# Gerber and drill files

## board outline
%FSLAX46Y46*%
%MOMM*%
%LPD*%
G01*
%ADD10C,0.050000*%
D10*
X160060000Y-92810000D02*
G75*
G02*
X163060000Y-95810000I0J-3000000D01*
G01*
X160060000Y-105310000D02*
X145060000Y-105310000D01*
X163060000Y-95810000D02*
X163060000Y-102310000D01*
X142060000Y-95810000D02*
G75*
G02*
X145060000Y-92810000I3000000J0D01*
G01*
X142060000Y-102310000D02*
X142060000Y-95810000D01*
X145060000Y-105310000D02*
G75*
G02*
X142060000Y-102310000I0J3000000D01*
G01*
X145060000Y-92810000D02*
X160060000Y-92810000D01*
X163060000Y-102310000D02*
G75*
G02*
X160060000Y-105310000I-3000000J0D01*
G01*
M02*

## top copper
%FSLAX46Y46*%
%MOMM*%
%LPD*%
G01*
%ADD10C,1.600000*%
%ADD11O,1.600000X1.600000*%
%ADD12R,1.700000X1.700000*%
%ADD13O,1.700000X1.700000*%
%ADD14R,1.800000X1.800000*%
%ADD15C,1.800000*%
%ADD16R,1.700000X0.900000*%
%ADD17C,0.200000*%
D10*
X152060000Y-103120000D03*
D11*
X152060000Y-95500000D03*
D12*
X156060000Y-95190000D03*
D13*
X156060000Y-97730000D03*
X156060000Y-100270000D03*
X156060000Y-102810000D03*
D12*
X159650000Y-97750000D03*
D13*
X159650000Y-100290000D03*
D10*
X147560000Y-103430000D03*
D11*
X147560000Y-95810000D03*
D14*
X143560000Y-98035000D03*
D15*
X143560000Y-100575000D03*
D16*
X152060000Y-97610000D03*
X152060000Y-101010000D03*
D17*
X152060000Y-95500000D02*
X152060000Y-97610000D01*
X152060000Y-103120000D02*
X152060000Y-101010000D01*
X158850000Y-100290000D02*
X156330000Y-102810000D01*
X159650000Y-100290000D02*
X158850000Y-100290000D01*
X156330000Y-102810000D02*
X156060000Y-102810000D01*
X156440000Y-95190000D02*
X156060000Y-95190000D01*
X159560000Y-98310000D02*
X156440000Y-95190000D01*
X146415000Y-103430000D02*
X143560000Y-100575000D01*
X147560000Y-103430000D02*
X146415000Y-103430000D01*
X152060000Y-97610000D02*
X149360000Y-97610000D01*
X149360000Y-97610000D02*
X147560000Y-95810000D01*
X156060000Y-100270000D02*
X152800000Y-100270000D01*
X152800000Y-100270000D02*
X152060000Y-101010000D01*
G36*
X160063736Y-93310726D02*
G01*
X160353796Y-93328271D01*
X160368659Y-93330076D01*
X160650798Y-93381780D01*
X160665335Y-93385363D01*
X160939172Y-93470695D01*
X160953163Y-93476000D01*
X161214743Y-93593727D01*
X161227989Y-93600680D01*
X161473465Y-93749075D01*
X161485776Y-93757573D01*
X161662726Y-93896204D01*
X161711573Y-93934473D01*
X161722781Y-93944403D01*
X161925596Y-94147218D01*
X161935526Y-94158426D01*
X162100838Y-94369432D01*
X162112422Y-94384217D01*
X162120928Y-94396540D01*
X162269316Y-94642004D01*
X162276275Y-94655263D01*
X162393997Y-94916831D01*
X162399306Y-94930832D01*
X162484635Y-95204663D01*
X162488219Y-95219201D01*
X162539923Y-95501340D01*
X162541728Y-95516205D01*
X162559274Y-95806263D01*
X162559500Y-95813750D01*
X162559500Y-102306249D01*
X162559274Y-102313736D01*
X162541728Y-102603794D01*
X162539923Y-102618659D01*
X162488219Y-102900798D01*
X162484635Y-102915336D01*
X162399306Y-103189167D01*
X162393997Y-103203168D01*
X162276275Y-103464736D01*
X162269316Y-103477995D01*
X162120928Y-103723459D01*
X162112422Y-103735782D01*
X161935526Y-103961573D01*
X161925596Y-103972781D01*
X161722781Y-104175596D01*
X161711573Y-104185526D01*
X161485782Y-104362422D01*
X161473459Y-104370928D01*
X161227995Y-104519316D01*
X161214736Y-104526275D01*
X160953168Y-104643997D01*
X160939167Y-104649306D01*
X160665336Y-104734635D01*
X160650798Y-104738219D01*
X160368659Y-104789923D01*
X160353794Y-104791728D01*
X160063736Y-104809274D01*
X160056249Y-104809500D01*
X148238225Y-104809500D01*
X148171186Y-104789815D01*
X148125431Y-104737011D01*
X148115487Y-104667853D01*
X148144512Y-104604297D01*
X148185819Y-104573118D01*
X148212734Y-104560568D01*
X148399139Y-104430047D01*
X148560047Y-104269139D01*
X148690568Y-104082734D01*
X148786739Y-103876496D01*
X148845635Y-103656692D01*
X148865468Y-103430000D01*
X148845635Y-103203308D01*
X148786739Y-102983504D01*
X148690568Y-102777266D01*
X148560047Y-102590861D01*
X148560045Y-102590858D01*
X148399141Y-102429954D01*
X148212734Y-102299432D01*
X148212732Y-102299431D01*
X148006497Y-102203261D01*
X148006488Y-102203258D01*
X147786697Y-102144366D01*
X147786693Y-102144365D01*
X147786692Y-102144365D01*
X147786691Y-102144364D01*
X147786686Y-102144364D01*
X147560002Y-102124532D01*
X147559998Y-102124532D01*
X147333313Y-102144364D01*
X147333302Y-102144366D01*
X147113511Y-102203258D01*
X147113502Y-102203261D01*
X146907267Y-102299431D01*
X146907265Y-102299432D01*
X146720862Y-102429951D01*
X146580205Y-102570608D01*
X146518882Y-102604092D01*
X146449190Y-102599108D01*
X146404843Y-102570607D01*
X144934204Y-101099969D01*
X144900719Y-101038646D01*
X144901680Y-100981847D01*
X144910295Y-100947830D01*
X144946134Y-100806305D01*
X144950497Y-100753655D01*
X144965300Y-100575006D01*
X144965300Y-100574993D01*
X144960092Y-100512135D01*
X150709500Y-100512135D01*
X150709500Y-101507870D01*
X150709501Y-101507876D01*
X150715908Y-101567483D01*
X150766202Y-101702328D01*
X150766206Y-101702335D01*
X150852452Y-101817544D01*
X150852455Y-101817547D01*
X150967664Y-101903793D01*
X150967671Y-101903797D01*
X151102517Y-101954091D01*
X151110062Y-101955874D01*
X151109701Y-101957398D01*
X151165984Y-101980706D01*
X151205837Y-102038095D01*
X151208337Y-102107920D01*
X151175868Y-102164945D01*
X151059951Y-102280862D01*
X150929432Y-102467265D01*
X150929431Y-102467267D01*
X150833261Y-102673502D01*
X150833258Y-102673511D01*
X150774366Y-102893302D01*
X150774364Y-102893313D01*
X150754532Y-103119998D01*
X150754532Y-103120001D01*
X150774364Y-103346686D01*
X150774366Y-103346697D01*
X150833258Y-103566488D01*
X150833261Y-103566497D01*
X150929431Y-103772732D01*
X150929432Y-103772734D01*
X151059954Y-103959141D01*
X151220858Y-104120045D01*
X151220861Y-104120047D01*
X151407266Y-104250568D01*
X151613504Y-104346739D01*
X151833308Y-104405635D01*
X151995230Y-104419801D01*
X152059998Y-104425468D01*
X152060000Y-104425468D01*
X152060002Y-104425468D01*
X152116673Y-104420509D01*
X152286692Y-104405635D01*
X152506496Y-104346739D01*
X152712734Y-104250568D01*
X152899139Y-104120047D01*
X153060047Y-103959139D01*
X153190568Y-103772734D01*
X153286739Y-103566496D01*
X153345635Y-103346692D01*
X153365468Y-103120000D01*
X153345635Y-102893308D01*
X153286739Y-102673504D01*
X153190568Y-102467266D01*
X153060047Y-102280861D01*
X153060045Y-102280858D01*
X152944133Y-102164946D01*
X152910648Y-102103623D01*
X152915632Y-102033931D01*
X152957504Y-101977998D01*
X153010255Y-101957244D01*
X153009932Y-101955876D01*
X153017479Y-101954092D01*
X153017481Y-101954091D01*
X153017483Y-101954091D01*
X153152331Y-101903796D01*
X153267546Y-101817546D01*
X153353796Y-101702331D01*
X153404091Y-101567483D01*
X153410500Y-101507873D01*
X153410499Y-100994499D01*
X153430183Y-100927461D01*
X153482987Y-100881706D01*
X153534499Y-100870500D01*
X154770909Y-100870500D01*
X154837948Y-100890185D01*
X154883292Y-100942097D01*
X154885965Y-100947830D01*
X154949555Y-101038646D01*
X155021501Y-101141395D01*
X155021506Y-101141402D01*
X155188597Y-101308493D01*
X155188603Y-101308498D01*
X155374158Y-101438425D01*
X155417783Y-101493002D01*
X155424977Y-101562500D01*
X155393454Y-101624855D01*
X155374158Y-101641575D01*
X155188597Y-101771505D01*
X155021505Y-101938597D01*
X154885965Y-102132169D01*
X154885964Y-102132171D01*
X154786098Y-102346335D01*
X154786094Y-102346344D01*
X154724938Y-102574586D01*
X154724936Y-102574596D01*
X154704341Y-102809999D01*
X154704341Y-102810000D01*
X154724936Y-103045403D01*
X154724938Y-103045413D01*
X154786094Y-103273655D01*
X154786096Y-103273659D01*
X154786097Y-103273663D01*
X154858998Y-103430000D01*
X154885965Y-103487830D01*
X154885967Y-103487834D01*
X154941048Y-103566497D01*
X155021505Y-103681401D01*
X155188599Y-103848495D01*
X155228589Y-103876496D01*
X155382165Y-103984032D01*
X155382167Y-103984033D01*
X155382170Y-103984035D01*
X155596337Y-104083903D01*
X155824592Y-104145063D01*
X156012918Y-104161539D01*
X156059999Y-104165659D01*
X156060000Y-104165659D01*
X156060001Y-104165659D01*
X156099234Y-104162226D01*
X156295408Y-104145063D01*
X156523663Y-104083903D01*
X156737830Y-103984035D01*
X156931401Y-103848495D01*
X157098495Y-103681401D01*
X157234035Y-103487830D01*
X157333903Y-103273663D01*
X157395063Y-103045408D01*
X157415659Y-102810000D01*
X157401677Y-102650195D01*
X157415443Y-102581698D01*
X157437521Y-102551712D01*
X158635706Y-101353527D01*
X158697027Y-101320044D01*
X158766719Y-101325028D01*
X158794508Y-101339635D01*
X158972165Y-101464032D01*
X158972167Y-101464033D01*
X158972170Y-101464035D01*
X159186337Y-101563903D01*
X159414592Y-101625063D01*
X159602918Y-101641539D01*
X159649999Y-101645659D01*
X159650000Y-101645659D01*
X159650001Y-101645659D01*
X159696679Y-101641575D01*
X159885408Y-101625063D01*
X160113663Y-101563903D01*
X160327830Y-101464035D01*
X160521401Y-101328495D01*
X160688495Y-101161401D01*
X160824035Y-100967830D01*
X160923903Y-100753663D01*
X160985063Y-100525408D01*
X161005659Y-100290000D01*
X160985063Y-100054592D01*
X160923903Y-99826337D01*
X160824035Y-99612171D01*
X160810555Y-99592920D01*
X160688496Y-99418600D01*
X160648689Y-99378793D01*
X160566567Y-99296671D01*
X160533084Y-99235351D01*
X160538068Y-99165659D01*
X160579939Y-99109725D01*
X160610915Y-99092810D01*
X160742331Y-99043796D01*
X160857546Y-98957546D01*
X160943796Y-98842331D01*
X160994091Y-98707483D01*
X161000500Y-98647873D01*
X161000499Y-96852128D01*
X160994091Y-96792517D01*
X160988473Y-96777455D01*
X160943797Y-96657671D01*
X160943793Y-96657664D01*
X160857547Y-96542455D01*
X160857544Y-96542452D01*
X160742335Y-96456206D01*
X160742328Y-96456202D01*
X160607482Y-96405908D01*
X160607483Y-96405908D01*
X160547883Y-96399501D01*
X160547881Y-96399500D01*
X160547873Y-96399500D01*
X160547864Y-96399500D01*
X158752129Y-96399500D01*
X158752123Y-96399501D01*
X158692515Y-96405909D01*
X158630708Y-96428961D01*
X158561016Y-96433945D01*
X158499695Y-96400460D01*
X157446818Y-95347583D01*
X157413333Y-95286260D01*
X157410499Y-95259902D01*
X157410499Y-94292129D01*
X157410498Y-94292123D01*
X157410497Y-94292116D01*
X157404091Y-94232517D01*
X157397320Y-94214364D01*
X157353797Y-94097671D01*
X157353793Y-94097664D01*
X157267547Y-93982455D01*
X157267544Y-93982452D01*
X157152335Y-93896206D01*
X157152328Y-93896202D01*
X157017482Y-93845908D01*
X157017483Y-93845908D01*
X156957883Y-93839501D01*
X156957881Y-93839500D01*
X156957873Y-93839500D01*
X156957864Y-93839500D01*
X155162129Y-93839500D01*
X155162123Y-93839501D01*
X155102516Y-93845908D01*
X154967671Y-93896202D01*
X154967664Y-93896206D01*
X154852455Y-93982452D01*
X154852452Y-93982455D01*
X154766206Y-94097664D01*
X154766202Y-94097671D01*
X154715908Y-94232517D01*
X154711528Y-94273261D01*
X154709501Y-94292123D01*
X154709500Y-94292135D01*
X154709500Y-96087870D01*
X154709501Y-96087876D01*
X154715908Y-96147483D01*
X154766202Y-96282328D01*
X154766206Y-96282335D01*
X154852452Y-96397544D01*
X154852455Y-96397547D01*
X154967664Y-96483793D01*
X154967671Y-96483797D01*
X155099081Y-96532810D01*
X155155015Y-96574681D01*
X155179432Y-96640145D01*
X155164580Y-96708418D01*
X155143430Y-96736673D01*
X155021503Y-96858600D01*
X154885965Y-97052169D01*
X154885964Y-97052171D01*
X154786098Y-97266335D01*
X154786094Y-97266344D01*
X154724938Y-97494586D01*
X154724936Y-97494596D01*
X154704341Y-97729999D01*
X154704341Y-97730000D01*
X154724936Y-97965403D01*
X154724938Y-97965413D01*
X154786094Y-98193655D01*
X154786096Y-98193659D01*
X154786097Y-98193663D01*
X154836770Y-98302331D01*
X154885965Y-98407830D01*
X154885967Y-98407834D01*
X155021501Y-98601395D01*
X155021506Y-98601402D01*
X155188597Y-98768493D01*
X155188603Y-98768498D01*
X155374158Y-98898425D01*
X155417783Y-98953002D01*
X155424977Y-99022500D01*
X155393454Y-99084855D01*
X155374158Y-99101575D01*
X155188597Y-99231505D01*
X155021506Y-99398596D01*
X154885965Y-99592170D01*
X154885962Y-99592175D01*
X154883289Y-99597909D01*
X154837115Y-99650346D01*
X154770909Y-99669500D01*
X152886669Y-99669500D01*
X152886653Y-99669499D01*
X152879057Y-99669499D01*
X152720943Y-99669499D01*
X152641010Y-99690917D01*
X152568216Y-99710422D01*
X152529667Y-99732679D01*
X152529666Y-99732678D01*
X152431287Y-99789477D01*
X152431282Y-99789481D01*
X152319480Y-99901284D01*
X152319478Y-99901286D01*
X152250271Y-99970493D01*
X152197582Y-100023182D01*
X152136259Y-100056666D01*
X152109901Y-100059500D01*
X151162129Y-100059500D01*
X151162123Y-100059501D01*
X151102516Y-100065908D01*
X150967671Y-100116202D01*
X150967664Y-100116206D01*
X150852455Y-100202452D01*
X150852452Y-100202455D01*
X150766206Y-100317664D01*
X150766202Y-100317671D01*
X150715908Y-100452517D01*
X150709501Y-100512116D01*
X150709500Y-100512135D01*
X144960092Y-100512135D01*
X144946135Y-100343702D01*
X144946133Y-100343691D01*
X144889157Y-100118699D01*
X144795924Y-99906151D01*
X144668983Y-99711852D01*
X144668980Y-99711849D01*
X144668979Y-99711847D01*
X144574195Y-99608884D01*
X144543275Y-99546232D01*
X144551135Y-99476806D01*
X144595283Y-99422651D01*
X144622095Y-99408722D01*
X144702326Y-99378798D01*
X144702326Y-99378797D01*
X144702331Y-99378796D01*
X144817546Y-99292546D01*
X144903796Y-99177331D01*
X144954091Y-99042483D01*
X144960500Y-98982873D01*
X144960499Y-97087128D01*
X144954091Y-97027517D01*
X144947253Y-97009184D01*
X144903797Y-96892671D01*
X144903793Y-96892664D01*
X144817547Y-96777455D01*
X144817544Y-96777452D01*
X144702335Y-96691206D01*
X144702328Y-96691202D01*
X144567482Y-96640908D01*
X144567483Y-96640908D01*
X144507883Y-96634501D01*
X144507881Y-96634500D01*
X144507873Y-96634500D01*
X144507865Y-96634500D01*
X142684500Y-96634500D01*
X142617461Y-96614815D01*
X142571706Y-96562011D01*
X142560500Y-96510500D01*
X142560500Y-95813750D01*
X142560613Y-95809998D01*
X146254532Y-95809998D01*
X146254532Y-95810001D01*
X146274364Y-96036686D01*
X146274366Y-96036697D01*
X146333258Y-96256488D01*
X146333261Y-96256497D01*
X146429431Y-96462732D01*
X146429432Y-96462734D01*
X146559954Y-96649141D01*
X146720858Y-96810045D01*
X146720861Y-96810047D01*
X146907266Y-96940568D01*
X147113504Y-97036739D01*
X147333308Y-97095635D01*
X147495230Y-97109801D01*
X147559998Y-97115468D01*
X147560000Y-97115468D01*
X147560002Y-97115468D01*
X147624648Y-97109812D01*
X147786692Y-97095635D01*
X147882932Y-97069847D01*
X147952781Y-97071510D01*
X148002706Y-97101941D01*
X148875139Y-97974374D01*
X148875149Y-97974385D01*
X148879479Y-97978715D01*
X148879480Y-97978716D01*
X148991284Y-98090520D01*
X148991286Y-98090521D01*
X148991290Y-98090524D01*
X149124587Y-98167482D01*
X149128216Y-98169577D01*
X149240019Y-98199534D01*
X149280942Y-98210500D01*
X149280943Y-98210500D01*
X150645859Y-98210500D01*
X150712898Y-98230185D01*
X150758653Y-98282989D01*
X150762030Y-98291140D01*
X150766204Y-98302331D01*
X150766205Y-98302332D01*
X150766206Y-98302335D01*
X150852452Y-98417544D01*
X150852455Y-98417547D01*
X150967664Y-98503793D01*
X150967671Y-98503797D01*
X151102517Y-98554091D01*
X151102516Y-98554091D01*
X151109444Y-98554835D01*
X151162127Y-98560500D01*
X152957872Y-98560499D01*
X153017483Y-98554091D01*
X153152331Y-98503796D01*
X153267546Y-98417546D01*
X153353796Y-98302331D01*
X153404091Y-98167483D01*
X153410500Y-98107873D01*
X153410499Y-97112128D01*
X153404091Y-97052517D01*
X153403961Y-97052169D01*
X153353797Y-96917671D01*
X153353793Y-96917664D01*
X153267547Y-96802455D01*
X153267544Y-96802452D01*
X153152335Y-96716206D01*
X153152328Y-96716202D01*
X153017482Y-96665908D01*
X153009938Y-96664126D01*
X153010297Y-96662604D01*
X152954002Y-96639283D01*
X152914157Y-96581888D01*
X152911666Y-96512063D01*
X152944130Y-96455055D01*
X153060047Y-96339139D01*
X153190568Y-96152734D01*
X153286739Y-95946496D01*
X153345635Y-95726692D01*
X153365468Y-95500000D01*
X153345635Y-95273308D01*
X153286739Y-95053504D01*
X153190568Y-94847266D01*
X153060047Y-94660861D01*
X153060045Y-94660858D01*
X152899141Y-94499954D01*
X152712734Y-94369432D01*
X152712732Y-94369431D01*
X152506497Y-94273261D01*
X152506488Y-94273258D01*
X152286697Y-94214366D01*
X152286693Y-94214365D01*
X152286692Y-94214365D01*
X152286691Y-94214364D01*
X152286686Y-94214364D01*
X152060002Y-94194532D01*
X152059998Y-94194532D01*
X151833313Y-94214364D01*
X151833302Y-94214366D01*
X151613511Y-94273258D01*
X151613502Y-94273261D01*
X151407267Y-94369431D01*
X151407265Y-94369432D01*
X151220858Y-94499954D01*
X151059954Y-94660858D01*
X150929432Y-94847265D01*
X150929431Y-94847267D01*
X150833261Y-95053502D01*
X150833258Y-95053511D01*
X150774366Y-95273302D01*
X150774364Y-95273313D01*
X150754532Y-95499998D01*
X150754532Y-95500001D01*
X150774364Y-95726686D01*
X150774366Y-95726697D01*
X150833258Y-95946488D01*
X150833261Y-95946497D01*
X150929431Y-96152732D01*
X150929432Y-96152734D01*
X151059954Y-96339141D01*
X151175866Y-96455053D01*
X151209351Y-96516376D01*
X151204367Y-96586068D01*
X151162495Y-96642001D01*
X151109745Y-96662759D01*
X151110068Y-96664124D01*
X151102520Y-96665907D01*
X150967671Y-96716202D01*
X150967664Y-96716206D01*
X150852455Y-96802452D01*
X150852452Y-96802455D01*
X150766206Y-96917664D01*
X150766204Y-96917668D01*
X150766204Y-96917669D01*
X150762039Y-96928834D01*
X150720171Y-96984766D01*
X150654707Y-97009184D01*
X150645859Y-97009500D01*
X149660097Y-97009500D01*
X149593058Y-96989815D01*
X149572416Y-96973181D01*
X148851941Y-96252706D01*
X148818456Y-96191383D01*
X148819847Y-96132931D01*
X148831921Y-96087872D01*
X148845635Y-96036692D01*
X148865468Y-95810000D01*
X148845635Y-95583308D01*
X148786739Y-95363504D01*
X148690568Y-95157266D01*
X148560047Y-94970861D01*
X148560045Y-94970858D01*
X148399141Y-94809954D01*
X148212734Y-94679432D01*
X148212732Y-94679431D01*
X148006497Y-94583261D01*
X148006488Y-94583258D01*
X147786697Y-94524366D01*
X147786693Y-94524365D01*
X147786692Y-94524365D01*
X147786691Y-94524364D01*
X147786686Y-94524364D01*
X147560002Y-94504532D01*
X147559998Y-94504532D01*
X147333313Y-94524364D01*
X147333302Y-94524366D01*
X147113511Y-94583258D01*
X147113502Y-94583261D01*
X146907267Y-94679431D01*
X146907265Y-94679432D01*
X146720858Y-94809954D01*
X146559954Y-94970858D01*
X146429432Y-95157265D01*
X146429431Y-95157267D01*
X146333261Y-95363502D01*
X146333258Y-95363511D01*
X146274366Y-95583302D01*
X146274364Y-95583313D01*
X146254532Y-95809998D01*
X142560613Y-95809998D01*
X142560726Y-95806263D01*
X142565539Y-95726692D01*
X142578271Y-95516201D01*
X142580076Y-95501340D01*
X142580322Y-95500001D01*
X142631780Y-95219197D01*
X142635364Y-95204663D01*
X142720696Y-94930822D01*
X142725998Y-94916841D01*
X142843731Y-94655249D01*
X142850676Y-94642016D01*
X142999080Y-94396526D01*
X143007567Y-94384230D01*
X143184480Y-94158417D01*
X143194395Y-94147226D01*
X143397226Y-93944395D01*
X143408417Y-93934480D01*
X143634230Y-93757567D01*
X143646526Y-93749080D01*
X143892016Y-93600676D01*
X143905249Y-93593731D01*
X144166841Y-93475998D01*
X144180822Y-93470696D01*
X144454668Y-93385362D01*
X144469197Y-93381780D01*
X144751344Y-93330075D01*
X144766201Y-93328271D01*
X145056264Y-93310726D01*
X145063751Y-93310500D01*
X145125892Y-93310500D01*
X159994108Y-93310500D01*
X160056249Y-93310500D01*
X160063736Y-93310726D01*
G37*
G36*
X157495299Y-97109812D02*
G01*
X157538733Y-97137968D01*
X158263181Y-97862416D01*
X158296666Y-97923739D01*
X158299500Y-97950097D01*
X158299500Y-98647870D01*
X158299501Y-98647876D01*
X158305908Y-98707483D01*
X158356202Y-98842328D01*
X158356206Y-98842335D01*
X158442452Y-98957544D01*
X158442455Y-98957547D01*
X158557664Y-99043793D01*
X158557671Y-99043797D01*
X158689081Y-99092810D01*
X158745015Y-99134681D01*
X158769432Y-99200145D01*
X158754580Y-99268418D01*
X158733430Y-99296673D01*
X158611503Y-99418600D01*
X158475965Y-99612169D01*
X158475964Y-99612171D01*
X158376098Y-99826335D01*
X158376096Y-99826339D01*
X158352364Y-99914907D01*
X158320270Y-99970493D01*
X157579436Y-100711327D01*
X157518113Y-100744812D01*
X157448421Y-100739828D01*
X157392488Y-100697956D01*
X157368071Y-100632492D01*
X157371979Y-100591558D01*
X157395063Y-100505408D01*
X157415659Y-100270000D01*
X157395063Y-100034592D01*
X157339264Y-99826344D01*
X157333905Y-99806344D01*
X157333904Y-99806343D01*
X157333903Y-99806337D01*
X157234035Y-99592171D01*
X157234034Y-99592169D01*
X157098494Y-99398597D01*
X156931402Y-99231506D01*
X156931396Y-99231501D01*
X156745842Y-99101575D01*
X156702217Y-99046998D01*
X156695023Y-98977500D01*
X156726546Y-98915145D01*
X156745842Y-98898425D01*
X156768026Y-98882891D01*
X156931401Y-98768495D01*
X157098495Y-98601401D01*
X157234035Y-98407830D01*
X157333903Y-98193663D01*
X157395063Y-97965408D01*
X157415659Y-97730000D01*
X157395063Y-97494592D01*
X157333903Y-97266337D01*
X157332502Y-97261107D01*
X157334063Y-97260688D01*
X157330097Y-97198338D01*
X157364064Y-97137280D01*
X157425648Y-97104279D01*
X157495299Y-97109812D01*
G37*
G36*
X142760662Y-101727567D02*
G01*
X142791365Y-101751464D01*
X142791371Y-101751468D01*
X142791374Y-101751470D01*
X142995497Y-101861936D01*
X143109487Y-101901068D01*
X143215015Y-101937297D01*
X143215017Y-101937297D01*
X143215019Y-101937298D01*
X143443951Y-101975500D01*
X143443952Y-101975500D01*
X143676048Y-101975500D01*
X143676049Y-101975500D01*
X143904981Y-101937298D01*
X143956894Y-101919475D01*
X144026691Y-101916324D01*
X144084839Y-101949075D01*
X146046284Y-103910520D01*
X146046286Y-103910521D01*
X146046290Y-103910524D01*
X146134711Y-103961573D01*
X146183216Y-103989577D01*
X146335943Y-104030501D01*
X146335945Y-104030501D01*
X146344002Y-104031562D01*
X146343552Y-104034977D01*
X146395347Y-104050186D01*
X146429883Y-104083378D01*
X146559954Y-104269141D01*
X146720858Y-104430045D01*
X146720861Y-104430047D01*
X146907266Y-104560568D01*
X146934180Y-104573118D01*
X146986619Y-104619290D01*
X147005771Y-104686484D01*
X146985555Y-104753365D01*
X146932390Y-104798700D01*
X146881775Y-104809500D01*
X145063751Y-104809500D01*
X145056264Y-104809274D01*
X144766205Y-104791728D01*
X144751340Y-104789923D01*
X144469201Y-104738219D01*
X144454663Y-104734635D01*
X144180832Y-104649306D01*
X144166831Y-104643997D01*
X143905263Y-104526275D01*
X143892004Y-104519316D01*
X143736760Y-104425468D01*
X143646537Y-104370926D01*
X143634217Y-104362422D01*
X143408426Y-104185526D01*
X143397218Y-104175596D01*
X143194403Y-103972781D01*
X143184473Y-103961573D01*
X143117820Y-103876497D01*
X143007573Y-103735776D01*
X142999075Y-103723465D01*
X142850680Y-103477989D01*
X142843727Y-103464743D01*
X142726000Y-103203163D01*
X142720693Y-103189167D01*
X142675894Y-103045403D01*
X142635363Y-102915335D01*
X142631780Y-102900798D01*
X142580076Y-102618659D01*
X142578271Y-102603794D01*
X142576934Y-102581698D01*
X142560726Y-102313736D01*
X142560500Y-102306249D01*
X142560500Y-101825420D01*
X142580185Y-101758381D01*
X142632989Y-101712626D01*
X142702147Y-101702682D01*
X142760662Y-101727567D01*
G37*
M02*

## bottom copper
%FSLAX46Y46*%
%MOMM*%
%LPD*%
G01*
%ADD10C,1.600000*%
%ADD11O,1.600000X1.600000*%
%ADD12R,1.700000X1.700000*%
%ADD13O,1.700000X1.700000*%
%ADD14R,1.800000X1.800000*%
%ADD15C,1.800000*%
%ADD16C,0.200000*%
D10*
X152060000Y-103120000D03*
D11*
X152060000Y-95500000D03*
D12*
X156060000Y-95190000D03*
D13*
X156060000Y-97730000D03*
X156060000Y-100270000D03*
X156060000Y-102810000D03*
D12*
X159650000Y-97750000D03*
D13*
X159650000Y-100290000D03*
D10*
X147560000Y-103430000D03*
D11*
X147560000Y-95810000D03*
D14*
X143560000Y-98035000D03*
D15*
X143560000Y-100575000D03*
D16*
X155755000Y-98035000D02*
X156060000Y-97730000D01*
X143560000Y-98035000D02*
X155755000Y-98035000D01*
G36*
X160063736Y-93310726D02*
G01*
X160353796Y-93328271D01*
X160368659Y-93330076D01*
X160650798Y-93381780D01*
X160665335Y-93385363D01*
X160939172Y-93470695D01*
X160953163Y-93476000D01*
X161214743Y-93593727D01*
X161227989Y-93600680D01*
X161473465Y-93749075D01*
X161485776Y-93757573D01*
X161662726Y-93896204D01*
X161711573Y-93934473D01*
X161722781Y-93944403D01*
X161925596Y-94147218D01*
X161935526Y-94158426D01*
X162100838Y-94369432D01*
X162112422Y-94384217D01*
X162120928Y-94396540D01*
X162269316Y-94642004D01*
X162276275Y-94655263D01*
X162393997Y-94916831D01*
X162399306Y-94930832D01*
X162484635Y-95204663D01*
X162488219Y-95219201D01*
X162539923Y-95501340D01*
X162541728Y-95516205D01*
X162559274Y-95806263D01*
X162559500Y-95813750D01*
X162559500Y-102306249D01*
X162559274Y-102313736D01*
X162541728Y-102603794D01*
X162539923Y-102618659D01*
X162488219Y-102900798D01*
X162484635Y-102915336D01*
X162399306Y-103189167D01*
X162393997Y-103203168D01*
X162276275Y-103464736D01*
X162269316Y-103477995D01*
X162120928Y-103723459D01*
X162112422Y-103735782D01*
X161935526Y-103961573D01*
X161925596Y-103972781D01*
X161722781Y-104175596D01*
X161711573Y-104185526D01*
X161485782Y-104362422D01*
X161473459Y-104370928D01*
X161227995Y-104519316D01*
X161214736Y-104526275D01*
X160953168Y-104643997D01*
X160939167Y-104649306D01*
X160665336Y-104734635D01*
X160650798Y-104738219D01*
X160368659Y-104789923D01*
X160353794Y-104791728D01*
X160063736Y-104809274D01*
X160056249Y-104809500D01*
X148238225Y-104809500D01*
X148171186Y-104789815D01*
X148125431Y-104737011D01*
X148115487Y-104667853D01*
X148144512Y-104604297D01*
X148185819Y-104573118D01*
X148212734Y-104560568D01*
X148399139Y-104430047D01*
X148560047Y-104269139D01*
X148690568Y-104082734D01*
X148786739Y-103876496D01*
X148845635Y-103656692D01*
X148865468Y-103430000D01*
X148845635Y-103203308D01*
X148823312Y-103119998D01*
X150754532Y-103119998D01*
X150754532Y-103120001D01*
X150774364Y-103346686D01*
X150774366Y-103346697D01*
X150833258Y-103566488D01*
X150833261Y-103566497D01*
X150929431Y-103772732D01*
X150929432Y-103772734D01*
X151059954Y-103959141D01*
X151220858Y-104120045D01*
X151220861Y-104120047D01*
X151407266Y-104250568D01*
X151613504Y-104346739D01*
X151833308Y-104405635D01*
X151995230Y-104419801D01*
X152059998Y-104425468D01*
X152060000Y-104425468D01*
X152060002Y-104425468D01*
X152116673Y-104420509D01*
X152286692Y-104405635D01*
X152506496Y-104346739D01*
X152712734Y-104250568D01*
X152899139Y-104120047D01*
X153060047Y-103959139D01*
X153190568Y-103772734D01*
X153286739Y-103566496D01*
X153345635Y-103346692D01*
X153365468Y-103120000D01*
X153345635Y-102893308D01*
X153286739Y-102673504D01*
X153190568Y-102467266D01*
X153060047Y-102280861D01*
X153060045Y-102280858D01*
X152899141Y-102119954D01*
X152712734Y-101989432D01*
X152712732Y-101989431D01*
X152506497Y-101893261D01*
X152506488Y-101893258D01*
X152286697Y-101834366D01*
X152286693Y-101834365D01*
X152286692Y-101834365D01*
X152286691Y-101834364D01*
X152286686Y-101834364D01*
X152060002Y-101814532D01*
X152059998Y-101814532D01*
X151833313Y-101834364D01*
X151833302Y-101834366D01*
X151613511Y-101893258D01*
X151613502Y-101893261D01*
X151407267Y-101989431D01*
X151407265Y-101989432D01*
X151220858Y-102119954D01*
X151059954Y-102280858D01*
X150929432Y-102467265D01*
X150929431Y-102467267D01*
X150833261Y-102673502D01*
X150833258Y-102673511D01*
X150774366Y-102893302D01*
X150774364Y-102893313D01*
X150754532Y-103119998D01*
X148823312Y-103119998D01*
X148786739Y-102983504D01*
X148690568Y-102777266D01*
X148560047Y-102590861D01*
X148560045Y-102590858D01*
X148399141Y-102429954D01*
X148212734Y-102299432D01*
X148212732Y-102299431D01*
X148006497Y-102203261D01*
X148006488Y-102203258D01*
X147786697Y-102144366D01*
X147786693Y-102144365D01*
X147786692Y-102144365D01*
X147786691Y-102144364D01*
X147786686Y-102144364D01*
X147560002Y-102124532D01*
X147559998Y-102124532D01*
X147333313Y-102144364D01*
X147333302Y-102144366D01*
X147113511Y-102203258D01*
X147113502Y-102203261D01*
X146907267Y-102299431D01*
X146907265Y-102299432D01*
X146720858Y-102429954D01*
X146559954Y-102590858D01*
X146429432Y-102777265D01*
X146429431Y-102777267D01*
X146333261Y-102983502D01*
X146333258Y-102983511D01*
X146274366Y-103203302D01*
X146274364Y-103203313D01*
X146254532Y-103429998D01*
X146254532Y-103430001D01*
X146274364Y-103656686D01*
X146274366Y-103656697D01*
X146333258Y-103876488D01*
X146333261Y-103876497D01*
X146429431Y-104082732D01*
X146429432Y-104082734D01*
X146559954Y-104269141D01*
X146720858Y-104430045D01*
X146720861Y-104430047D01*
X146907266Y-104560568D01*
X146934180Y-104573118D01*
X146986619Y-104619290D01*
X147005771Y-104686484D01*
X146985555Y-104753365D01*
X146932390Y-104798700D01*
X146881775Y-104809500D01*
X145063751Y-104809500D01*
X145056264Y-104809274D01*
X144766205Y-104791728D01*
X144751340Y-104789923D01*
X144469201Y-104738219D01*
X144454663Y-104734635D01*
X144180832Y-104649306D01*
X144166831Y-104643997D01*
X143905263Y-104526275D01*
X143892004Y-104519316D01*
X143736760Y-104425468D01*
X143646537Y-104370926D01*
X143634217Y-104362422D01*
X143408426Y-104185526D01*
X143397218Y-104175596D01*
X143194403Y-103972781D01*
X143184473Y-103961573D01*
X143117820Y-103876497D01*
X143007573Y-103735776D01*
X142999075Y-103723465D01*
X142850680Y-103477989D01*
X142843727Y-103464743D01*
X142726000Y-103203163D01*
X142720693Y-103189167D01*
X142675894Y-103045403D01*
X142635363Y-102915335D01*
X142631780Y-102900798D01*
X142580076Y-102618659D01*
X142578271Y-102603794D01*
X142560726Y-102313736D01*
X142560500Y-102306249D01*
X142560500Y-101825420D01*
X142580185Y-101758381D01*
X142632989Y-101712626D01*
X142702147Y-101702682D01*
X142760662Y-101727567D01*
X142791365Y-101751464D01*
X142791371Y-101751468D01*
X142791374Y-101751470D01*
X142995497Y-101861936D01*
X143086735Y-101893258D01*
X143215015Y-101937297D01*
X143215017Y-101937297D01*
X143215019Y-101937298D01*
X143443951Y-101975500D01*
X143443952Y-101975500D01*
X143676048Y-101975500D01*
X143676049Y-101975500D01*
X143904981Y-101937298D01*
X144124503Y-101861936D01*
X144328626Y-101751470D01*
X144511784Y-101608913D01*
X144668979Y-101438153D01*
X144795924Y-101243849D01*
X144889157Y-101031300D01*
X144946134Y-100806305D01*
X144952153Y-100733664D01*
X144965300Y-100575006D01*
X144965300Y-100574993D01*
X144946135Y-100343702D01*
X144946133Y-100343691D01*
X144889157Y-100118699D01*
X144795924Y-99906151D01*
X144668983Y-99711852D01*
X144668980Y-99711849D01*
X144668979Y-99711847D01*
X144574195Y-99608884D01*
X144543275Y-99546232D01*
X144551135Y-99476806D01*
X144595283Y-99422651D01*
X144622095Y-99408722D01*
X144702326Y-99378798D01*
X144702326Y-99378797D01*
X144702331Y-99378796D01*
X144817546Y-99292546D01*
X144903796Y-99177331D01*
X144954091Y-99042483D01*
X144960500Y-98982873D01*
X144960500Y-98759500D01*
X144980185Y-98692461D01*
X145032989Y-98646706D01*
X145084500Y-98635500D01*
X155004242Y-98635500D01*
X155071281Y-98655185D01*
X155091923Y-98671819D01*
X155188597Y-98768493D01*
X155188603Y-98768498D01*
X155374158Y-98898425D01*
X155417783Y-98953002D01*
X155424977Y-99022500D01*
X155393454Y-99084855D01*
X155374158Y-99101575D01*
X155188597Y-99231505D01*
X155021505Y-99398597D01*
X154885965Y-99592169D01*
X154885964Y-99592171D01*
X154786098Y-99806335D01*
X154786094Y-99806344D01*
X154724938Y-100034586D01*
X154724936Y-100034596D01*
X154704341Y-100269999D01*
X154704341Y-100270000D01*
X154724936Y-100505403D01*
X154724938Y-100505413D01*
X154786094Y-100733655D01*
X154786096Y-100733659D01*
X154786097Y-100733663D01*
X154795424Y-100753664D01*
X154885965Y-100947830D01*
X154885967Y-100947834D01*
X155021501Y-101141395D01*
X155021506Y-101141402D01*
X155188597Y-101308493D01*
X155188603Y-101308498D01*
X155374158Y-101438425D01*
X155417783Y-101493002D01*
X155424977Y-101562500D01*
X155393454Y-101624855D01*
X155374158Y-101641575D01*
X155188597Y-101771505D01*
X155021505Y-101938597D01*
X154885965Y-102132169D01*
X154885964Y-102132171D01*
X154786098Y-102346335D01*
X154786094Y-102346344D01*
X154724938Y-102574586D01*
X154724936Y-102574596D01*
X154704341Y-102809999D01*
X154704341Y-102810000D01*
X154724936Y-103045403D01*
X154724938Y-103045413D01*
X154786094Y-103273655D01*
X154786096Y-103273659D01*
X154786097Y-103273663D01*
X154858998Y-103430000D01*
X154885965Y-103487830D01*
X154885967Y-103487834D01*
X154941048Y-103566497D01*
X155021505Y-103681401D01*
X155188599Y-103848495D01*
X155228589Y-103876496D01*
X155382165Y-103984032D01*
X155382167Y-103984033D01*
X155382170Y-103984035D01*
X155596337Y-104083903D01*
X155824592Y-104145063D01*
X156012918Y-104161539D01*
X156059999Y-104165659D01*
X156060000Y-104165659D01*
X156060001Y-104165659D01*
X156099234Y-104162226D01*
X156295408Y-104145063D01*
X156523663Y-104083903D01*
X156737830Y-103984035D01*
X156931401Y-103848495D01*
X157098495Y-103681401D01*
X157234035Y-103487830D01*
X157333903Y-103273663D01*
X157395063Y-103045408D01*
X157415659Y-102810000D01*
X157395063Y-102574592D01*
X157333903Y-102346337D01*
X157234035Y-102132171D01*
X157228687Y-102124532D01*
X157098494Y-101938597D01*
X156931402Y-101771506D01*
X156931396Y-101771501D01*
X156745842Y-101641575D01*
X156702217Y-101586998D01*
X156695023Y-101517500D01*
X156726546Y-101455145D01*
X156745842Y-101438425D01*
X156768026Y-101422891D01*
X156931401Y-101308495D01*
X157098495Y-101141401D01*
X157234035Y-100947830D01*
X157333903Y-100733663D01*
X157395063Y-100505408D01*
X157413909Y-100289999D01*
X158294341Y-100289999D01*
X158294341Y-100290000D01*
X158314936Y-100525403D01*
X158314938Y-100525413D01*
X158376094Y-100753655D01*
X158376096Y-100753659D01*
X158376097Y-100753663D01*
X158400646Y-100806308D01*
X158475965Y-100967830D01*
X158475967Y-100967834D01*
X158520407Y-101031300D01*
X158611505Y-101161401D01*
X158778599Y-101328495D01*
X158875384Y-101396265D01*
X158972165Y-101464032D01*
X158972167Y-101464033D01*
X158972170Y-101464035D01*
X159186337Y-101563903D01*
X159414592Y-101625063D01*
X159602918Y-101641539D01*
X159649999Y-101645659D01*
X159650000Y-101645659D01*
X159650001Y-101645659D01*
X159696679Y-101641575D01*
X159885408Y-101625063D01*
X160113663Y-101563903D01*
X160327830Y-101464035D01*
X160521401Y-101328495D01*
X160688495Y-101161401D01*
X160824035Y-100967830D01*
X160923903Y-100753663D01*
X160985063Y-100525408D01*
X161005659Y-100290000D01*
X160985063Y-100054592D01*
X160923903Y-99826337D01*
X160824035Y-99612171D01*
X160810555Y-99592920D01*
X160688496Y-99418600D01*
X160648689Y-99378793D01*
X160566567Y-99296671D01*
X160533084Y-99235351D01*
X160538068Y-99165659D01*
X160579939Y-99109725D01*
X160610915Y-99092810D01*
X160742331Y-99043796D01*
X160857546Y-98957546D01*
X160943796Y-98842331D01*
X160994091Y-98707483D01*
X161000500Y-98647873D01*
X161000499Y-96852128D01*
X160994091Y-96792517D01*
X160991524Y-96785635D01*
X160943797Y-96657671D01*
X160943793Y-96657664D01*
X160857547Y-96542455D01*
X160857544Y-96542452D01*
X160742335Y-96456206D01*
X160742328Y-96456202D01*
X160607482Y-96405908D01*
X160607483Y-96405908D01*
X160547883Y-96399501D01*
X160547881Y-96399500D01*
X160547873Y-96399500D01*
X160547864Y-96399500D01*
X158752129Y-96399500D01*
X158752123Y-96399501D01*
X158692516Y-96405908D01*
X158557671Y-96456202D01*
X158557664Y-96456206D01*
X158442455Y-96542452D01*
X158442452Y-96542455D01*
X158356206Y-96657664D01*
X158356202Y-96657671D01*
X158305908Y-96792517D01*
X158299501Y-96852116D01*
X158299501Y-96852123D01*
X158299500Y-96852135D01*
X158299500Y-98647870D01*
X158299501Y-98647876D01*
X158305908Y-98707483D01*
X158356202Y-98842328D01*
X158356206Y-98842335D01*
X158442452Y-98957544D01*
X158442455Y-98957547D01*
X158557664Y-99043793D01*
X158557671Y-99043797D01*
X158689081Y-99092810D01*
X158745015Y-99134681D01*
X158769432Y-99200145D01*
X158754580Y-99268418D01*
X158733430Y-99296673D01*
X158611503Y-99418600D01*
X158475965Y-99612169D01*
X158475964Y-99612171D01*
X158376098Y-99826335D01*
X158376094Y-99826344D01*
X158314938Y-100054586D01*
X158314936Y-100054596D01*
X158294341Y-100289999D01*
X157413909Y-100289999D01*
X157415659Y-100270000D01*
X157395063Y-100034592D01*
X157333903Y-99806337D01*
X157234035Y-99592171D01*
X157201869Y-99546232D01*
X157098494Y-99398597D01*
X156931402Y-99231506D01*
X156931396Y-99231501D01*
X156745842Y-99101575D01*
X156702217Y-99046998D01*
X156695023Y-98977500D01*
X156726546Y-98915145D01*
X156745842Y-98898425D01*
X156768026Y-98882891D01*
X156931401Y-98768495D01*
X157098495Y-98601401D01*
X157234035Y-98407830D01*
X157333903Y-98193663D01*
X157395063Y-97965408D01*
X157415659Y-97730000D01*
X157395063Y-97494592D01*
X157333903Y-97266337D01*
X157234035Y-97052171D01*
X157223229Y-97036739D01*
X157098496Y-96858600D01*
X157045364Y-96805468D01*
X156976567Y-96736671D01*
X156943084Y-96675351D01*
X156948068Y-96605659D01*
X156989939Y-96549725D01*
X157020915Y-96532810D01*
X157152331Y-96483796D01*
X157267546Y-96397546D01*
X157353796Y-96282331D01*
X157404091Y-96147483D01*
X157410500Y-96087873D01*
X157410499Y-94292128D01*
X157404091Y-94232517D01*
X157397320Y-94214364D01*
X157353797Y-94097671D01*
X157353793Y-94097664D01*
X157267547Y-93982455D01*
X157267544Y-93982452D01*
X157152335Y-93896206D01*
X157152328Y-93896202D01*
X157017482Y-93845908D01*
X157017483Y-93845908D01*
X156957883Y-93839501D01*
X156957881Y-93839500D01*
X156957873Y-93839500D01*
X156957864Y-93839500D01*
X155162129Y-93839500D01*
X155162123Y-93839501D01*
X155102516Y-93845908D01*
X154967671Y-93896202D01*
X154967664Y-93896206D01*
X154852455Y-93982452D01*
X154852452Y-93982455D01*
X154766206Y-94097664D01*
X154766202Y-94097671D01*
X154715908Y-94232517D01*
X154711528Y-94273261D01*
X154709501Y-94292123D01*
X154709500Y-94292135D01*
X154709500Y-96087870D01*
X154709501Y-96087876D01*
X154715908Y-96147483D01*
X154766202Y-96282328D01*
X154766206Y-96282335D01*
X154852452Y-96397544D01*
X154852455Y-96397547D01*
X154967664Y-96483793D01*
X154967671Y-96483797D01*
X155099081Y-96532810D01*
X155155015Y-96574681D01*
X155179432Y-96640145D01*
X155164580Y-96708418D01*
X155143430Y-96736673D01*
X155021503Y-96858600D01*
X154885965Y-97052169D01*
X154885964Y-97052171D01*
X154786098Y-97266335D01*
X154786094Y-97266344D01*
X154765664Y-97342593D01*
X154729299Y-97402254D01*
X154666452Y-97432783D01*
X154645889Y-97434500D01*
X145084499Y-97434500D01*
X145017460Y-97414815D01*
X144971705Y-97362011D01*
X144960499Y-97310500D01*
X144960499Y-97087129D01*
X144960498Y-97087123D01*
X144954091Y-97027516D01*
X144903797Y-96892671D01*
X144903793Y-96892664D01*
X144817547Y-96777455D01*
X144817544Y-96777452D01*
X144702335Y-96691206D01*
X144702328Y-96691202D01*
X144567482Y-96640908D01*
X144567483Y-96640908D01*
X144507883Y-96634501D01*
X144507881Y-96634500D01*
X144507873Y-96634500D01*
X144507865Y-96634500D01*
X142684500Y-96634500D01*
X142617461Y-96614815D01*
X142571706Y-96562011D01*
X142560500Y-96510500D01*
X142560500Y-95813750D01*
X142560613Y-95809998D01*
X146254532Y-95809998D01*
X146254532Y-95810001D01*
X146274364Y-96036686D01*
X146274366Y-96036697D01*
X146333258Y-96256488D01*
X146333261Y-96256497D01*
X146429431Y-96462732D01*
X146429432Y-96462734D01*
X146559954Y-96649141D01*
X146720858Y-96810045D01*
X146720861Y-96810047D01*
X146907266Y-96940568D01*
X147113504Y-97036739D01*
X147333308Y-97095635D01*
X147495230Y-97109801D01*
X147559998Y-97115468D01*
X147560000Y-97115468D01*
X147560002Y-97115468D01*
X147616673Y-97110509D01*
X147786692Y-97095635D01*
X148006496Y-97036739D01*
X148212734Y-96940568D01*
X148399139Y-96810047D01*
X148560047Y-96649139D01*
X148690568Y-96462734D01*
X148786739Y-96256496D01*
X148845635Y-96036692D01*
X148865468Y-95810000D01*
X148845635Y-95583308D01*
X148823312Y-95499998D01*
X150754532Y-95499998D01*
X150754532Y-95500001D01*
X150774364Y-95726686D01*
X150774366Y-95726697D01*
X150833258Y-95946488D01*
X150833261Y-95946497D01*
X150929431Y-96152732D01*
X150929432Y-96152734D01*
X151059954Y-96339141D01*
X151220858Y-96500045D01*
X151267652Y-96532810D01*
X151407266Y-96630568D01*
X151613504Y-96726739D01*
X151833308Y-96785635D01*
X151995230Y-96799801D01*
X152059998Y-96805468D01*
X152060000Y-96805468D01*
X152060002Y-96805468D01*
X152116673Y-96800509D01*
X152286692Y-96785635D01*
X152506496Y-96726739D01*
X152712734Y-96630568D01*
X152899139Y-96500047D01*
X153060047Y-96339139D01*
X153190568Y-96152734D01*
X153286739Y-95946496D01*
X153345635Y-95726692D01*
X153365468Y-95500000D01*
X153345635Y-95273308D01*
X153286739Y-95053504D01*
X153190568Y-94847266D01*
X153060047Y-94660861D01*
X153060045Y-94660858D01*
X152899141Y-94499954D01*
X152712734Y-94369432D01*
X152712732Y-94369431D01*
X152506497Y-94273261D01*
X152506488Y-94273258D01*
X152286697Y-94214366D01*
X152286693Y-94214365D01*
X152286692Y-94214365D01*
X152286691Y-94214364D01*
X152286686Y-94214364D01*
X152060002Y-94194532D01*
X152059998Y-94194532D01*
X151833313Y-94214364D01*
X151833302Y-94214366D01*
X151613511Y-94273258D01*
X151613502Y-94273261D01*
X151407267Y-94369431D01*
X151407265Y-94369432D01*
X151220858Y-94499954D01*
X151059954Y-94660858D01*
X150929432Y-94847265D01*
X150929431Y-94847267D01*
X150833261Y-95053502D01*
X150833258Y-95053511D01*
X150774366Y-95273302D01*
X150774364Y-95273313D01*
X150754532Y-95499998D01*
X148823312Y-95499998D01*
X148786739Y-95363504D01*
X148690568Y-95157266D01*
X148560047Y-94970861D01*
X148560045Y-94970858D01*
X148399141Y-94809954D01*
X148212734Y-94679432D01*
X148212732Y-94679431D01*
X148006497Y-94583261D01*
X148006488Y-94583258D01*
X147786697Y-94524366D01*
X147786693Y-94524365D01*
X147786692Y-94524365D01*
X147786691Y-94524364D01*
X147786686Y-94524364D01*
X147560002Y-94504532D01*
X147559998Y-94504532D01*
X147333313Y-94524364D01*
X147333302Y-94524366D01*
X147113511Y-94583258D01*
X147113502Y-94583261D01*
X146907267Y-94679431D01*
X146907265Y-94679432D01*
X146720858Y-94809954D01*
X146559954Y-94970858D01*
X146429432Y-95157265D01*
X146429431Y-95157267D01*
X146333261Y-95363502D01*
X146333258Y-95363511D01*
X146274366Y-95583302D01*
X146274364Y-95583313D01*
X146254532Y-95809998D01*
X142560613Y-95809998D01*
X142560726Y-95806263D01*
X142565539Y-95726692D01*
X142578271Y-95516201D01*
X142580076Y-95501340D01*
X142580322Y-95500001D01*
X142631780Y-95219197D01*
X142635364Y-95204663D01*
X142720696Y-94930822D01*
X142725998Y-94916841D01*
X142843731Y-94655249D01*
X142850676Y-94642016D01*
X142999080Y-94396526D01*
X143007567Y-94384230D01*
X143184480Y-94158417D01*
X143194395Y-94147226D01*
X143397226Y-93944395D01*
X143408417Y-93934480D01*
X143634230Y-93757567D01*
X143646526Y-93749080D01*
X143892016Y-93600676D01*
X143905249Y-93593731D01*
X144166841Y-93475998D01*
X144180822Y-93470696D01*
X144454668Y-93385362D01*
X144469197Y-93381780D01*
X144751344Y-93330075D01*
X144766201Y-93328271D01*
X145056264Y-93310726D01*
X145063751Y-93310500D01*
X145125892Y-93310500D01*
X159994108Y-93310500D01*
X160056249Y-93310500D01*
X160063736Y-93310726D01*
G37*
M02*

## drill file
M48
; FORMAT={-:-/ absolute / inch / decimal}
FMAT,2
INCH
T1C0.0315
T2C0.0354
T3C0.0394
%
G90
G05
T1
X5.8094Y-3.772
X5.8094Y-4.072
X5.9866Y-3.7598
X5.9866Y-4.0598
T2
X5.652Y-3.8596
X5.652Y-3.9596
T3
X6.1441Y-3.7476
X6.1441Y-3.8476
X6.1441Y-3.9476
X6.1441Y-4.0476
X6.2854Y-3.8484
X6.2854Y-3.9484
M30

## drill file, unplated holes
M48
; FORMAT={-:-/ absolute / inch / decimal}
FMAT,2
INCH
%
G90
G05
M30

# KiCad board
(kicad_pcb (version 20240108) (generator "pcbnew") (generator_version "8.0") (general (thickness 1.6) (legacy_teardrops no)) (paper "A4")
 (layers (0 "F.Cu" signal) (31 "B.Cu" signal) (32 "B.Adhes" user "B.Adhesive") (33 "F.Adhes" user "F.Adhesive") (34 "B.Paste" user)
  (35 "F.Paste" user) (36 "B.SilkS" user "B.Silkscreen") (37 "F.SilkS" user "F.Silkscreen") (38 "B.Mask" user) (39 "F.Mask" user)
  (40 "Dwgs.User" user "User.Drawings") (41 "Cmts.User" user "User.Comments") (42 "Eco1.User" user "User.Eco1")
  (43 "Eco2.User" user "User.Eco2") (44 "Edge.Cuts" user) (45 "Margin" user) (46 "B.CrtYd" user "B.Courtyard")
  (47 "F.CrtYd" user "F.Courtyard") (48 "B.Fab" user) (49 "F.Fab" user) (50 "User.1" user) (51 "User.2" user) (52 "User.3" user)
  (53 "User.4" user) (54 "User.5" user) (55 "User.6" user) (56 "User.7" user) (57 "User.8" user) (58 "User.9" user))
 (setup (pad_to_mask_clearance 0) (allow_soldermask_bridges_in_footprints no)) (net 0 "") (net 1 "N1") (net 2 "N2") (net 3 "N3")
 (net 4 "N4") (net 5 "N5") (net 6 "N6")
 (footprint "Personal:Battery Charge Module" (layer "F.Cu") (at 156.06 98.77)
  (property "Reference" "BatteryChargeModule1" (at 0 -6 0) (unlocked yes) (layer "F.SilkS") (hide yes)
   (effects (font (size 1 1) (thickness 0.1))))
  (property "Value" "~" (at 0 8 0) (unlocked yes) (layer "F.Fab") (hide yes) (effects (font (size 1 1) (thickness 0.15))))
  (pad "1" thru_hole rect (at 0 -3.58) (size 1.7 1.7) (drill 1) (layers "*.Cu" "*.Mask") (remove_unused_layers no) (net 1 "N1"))
  (pad "2" thru_hole oval (at 0 -1.04) (size 1.7 1.7) (drill 1) (layers "*.Cu" "*.Mask") (remove_unused_layers no) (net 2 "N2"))
  (pad "3" thru_hole oval (at 0 1.5) (size 1.7 1.7) (drill 1) (layers "*.Cu" "*.Mask") (remove_unused_layers no) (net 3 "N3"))
  (pad "4" thru_hole oval (at 0 4.04) (size 1.7 1.7) (drill 1) (layers "*.Cu" "*.Mask") (remove_unused_layers no) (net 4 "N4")))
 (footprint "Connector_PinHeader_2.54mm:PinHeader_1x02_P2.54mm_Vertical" (layer "F.Cu") (at 159.65 97.75)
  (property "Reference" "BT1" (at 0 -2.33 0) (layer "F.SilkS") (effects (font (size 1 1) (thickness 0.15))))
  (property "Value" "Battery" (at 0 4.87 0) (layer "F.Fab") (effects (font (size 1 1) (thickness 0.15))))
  (pad "1" thru_hole rect (at 0 0) (size 1.7 1.7) (drill 1) (layers "*.Cu" "*.Mask") (remove_unused_layers no) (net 1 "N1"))
  (pad "2" thru_hole oval (at 0 2.54) (size 1.7 1.7) (drill 1) (layers "*.Cu" "*.Mask") (remove_unused_layers no) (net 4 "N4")))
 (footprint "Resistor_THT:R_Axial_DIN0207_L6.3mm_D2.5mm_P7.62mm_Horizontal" (layer "F.Cu") (at 147.56 103.43 90)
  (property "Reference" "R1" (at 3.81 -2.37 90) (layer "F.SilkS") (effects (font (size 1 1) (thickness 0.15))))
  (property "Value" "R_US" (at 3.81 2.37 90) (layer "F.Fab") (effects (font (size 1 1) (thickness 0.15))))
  (pad "1" thru_hole circle (at 0 0 90) (size 1.6 1.6) (drill 0.8) (layers "*.Cu" "*.Mask") (remove_unused_layers no) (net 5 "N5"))
  (pad "2" thru_hole oval (at 7.62 0 90) (size 1.6 1.6) (drill 0.8) (layers "*.Cu" "*.Mask") (remove_unused_layers no) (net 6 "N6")))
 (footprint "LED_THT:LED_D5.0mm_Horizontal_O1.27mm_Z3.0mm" (layer "F.Cu") (at 143.56 98.035 -90)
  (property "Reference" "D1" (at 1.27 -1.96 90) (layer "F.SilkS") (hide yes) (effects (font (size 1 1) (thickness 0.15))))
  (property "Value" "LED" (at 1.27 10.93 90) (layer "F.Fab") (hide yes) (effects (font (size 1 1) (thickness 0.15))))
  (pad "1" thru_hole rect (at 0 0 270) (size 1.8 1.8) (drill 0.9) (layers "*.Cu" "*.Mask") (remove_unused_layers no) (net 2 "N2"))
  (pad "2" thru_hole circle (at 2.54 0 270) (size 1.8 1.8) (drill 0.9) (layers "*.Cu" "*.Mask") (remove_unused_layers no) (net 5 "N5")))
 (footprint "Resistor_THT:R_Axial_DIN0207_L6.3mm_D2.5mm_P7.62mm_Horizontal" (layer "F.Cu") (at 152.06 103.12 90)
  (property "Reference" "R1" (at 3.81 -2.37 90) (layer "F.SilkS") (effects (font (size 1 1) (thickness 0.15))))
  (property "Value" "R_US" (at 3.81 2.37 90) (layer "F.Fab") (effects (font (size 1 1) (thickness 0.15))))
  (pad "1" thru_hole circle (at 0 0 90) (size 1.6 1.6) (drill 0.8) (layers "*.Cu" "*.Mask") (remove_unused_layers no) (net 3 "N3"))
  (pad "2" thru_hole oval (at 7.62 0 90) (size 1.6 1.6) (drill 0.8) (layers "*.Cu" "*.Mask") (remove_unused_layers no) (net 6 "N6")))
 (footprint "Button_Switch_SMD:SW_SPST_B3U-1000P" (layer "F.Cu") (at 152.06 99.31 -90)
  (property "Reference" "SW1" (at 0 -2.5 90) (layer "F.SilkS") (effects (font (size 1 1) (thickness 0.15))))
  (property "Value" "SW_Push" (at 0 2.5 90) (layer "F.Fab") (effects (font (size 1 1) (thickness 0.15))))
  (pad "1" smd rect (at -1.7 0 270) (size 0.9 1.7) (layers "F.Cu" "F.Paste" "F.Mask") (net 6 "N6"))
  (pad "2" smd rect (at 1.7 0 270) (size 0.9 1.7) (layers "F.Cu" "F.Paste" "F.Mask") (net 3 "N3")))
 (gr_arc (start 160.06 92.81) (mid 162.18132 93.68868) (end 163.06 95.81) (stroke (width 0.05) (type default)) (layer "Edge.Cuts"))
 (gr_line (start 160.06 105.31) (end 145.06 105.31) (stroke (width 0.05) (type default)) (layer "Edge.Cuts"))
 (gr_line (start 163.06 95.81) (end 163.06 102.31) (stroke (width 0.05) (type default)) (layer "Edge.Cuts"))
 (gr_arc (start 142.06 95.81) (mid 142.93868 93.68868) (end 145.06 92.81) (stroke (width 0.05) (type default)) (layer "Edge.Cuts"))
 (gr_line (start 142.06 102.31) (end 142.06 95.81) (stroke (width 0.05) (type default)) (layer "Edge.Cuts"))
 (gr_arc (start 145.06 105.31) (mid 142.93868 104.43132) (end 142.06 102.31) (stroke (width 0.05) (type default)) (layer "Edge.Cuts"))
 (gr_line (start 145.06 92.81) (end 160.06 92.81) (stroke (width 0.05) (type default)) (layer "Edge.Cuts"))
 (gr_arc (start 163.06 102.31) (mid 162.18132 104.43132) (end 160.06 105.31) (stroke (width 0.05) (type default)) (layer "Edge.Cuts"))
 (segment (start 158.85 100.29) (end 156.33 102.81) (width 0.2) (layer "F.Cu") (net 4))
 (segment (start 159.65 100.29) (end 158.85 100.29) (width 0.2) (layer "F.Cu") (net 4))
 (segment (start 156.33 102.81) (end 156.06 102.81) (width 0.2) (layer "F.Cu") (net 4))
 (segment (start 156.44 95.19) (end 156.06 95.19) (width 0.2) (layer "F.Cu") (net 1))
 (segment (start 159.56 98.31) (end 156.44 95.19) (width 0.2) (layer "F.Cu") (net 1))
 (segment (start 146.415 103.43) (end 143.56 100.575) (width 0.2) (layer "F.Cu") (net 5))
 (segment (start 147.56 103.43) (end 146.415 103.43) (width 0.2) (layer "F.Cu") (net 5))
 (segment (start 152.06 97.61) (end 149.36 97.61) (width 0.2) (layer "F.Cu") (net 6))
 (segment (start 149.36 97.61) (end 147.56 95.81) (width 0.2) (layer "F.Cu") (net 6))
 (segment (start 152.06 95.5) (end 152.06 97.61) (width 0.2) (layer "F.Cu") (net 6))
 (segment (start 155.755 98.035) (end 156.06 97.73) (width 0.2) (layer "B.Cu") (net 2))
 (segment (start 143.56 98.035) (end 155.755 98.035) (width 0.2) (layer "B.Cu") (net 2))
 (segment (start 152.06 103.12) (end 152.06 101.01) (width 0.2) (layer "F.Cu") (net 3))
 (segment (start 156.06 100.27) (end 152.8 100.27) (width 0.2) (layer "F.Cu") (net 3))
 (segment (start 152.8 100.27) (end 152.06 101.01) (width 0.2) (layer "F.Cu") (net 3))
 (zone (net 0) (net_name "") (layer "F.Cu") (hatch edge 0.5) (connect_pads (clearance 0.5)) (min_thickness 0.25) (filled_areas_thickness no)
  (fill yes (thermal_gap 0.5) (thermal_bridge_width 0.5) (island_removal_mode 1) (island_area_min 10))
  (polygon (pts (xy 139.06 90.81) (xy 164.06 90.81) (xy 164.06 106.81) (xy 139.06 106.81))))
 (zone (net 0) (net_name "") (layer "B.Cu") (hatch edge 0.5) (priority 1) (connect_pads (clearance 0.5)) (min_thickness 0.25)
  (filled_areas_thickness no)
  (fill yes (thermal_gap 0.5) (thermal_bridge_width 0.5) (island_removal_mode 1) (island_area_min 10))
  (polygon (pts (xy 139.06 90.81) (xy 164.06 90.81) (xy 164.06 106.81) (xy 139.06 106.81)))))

